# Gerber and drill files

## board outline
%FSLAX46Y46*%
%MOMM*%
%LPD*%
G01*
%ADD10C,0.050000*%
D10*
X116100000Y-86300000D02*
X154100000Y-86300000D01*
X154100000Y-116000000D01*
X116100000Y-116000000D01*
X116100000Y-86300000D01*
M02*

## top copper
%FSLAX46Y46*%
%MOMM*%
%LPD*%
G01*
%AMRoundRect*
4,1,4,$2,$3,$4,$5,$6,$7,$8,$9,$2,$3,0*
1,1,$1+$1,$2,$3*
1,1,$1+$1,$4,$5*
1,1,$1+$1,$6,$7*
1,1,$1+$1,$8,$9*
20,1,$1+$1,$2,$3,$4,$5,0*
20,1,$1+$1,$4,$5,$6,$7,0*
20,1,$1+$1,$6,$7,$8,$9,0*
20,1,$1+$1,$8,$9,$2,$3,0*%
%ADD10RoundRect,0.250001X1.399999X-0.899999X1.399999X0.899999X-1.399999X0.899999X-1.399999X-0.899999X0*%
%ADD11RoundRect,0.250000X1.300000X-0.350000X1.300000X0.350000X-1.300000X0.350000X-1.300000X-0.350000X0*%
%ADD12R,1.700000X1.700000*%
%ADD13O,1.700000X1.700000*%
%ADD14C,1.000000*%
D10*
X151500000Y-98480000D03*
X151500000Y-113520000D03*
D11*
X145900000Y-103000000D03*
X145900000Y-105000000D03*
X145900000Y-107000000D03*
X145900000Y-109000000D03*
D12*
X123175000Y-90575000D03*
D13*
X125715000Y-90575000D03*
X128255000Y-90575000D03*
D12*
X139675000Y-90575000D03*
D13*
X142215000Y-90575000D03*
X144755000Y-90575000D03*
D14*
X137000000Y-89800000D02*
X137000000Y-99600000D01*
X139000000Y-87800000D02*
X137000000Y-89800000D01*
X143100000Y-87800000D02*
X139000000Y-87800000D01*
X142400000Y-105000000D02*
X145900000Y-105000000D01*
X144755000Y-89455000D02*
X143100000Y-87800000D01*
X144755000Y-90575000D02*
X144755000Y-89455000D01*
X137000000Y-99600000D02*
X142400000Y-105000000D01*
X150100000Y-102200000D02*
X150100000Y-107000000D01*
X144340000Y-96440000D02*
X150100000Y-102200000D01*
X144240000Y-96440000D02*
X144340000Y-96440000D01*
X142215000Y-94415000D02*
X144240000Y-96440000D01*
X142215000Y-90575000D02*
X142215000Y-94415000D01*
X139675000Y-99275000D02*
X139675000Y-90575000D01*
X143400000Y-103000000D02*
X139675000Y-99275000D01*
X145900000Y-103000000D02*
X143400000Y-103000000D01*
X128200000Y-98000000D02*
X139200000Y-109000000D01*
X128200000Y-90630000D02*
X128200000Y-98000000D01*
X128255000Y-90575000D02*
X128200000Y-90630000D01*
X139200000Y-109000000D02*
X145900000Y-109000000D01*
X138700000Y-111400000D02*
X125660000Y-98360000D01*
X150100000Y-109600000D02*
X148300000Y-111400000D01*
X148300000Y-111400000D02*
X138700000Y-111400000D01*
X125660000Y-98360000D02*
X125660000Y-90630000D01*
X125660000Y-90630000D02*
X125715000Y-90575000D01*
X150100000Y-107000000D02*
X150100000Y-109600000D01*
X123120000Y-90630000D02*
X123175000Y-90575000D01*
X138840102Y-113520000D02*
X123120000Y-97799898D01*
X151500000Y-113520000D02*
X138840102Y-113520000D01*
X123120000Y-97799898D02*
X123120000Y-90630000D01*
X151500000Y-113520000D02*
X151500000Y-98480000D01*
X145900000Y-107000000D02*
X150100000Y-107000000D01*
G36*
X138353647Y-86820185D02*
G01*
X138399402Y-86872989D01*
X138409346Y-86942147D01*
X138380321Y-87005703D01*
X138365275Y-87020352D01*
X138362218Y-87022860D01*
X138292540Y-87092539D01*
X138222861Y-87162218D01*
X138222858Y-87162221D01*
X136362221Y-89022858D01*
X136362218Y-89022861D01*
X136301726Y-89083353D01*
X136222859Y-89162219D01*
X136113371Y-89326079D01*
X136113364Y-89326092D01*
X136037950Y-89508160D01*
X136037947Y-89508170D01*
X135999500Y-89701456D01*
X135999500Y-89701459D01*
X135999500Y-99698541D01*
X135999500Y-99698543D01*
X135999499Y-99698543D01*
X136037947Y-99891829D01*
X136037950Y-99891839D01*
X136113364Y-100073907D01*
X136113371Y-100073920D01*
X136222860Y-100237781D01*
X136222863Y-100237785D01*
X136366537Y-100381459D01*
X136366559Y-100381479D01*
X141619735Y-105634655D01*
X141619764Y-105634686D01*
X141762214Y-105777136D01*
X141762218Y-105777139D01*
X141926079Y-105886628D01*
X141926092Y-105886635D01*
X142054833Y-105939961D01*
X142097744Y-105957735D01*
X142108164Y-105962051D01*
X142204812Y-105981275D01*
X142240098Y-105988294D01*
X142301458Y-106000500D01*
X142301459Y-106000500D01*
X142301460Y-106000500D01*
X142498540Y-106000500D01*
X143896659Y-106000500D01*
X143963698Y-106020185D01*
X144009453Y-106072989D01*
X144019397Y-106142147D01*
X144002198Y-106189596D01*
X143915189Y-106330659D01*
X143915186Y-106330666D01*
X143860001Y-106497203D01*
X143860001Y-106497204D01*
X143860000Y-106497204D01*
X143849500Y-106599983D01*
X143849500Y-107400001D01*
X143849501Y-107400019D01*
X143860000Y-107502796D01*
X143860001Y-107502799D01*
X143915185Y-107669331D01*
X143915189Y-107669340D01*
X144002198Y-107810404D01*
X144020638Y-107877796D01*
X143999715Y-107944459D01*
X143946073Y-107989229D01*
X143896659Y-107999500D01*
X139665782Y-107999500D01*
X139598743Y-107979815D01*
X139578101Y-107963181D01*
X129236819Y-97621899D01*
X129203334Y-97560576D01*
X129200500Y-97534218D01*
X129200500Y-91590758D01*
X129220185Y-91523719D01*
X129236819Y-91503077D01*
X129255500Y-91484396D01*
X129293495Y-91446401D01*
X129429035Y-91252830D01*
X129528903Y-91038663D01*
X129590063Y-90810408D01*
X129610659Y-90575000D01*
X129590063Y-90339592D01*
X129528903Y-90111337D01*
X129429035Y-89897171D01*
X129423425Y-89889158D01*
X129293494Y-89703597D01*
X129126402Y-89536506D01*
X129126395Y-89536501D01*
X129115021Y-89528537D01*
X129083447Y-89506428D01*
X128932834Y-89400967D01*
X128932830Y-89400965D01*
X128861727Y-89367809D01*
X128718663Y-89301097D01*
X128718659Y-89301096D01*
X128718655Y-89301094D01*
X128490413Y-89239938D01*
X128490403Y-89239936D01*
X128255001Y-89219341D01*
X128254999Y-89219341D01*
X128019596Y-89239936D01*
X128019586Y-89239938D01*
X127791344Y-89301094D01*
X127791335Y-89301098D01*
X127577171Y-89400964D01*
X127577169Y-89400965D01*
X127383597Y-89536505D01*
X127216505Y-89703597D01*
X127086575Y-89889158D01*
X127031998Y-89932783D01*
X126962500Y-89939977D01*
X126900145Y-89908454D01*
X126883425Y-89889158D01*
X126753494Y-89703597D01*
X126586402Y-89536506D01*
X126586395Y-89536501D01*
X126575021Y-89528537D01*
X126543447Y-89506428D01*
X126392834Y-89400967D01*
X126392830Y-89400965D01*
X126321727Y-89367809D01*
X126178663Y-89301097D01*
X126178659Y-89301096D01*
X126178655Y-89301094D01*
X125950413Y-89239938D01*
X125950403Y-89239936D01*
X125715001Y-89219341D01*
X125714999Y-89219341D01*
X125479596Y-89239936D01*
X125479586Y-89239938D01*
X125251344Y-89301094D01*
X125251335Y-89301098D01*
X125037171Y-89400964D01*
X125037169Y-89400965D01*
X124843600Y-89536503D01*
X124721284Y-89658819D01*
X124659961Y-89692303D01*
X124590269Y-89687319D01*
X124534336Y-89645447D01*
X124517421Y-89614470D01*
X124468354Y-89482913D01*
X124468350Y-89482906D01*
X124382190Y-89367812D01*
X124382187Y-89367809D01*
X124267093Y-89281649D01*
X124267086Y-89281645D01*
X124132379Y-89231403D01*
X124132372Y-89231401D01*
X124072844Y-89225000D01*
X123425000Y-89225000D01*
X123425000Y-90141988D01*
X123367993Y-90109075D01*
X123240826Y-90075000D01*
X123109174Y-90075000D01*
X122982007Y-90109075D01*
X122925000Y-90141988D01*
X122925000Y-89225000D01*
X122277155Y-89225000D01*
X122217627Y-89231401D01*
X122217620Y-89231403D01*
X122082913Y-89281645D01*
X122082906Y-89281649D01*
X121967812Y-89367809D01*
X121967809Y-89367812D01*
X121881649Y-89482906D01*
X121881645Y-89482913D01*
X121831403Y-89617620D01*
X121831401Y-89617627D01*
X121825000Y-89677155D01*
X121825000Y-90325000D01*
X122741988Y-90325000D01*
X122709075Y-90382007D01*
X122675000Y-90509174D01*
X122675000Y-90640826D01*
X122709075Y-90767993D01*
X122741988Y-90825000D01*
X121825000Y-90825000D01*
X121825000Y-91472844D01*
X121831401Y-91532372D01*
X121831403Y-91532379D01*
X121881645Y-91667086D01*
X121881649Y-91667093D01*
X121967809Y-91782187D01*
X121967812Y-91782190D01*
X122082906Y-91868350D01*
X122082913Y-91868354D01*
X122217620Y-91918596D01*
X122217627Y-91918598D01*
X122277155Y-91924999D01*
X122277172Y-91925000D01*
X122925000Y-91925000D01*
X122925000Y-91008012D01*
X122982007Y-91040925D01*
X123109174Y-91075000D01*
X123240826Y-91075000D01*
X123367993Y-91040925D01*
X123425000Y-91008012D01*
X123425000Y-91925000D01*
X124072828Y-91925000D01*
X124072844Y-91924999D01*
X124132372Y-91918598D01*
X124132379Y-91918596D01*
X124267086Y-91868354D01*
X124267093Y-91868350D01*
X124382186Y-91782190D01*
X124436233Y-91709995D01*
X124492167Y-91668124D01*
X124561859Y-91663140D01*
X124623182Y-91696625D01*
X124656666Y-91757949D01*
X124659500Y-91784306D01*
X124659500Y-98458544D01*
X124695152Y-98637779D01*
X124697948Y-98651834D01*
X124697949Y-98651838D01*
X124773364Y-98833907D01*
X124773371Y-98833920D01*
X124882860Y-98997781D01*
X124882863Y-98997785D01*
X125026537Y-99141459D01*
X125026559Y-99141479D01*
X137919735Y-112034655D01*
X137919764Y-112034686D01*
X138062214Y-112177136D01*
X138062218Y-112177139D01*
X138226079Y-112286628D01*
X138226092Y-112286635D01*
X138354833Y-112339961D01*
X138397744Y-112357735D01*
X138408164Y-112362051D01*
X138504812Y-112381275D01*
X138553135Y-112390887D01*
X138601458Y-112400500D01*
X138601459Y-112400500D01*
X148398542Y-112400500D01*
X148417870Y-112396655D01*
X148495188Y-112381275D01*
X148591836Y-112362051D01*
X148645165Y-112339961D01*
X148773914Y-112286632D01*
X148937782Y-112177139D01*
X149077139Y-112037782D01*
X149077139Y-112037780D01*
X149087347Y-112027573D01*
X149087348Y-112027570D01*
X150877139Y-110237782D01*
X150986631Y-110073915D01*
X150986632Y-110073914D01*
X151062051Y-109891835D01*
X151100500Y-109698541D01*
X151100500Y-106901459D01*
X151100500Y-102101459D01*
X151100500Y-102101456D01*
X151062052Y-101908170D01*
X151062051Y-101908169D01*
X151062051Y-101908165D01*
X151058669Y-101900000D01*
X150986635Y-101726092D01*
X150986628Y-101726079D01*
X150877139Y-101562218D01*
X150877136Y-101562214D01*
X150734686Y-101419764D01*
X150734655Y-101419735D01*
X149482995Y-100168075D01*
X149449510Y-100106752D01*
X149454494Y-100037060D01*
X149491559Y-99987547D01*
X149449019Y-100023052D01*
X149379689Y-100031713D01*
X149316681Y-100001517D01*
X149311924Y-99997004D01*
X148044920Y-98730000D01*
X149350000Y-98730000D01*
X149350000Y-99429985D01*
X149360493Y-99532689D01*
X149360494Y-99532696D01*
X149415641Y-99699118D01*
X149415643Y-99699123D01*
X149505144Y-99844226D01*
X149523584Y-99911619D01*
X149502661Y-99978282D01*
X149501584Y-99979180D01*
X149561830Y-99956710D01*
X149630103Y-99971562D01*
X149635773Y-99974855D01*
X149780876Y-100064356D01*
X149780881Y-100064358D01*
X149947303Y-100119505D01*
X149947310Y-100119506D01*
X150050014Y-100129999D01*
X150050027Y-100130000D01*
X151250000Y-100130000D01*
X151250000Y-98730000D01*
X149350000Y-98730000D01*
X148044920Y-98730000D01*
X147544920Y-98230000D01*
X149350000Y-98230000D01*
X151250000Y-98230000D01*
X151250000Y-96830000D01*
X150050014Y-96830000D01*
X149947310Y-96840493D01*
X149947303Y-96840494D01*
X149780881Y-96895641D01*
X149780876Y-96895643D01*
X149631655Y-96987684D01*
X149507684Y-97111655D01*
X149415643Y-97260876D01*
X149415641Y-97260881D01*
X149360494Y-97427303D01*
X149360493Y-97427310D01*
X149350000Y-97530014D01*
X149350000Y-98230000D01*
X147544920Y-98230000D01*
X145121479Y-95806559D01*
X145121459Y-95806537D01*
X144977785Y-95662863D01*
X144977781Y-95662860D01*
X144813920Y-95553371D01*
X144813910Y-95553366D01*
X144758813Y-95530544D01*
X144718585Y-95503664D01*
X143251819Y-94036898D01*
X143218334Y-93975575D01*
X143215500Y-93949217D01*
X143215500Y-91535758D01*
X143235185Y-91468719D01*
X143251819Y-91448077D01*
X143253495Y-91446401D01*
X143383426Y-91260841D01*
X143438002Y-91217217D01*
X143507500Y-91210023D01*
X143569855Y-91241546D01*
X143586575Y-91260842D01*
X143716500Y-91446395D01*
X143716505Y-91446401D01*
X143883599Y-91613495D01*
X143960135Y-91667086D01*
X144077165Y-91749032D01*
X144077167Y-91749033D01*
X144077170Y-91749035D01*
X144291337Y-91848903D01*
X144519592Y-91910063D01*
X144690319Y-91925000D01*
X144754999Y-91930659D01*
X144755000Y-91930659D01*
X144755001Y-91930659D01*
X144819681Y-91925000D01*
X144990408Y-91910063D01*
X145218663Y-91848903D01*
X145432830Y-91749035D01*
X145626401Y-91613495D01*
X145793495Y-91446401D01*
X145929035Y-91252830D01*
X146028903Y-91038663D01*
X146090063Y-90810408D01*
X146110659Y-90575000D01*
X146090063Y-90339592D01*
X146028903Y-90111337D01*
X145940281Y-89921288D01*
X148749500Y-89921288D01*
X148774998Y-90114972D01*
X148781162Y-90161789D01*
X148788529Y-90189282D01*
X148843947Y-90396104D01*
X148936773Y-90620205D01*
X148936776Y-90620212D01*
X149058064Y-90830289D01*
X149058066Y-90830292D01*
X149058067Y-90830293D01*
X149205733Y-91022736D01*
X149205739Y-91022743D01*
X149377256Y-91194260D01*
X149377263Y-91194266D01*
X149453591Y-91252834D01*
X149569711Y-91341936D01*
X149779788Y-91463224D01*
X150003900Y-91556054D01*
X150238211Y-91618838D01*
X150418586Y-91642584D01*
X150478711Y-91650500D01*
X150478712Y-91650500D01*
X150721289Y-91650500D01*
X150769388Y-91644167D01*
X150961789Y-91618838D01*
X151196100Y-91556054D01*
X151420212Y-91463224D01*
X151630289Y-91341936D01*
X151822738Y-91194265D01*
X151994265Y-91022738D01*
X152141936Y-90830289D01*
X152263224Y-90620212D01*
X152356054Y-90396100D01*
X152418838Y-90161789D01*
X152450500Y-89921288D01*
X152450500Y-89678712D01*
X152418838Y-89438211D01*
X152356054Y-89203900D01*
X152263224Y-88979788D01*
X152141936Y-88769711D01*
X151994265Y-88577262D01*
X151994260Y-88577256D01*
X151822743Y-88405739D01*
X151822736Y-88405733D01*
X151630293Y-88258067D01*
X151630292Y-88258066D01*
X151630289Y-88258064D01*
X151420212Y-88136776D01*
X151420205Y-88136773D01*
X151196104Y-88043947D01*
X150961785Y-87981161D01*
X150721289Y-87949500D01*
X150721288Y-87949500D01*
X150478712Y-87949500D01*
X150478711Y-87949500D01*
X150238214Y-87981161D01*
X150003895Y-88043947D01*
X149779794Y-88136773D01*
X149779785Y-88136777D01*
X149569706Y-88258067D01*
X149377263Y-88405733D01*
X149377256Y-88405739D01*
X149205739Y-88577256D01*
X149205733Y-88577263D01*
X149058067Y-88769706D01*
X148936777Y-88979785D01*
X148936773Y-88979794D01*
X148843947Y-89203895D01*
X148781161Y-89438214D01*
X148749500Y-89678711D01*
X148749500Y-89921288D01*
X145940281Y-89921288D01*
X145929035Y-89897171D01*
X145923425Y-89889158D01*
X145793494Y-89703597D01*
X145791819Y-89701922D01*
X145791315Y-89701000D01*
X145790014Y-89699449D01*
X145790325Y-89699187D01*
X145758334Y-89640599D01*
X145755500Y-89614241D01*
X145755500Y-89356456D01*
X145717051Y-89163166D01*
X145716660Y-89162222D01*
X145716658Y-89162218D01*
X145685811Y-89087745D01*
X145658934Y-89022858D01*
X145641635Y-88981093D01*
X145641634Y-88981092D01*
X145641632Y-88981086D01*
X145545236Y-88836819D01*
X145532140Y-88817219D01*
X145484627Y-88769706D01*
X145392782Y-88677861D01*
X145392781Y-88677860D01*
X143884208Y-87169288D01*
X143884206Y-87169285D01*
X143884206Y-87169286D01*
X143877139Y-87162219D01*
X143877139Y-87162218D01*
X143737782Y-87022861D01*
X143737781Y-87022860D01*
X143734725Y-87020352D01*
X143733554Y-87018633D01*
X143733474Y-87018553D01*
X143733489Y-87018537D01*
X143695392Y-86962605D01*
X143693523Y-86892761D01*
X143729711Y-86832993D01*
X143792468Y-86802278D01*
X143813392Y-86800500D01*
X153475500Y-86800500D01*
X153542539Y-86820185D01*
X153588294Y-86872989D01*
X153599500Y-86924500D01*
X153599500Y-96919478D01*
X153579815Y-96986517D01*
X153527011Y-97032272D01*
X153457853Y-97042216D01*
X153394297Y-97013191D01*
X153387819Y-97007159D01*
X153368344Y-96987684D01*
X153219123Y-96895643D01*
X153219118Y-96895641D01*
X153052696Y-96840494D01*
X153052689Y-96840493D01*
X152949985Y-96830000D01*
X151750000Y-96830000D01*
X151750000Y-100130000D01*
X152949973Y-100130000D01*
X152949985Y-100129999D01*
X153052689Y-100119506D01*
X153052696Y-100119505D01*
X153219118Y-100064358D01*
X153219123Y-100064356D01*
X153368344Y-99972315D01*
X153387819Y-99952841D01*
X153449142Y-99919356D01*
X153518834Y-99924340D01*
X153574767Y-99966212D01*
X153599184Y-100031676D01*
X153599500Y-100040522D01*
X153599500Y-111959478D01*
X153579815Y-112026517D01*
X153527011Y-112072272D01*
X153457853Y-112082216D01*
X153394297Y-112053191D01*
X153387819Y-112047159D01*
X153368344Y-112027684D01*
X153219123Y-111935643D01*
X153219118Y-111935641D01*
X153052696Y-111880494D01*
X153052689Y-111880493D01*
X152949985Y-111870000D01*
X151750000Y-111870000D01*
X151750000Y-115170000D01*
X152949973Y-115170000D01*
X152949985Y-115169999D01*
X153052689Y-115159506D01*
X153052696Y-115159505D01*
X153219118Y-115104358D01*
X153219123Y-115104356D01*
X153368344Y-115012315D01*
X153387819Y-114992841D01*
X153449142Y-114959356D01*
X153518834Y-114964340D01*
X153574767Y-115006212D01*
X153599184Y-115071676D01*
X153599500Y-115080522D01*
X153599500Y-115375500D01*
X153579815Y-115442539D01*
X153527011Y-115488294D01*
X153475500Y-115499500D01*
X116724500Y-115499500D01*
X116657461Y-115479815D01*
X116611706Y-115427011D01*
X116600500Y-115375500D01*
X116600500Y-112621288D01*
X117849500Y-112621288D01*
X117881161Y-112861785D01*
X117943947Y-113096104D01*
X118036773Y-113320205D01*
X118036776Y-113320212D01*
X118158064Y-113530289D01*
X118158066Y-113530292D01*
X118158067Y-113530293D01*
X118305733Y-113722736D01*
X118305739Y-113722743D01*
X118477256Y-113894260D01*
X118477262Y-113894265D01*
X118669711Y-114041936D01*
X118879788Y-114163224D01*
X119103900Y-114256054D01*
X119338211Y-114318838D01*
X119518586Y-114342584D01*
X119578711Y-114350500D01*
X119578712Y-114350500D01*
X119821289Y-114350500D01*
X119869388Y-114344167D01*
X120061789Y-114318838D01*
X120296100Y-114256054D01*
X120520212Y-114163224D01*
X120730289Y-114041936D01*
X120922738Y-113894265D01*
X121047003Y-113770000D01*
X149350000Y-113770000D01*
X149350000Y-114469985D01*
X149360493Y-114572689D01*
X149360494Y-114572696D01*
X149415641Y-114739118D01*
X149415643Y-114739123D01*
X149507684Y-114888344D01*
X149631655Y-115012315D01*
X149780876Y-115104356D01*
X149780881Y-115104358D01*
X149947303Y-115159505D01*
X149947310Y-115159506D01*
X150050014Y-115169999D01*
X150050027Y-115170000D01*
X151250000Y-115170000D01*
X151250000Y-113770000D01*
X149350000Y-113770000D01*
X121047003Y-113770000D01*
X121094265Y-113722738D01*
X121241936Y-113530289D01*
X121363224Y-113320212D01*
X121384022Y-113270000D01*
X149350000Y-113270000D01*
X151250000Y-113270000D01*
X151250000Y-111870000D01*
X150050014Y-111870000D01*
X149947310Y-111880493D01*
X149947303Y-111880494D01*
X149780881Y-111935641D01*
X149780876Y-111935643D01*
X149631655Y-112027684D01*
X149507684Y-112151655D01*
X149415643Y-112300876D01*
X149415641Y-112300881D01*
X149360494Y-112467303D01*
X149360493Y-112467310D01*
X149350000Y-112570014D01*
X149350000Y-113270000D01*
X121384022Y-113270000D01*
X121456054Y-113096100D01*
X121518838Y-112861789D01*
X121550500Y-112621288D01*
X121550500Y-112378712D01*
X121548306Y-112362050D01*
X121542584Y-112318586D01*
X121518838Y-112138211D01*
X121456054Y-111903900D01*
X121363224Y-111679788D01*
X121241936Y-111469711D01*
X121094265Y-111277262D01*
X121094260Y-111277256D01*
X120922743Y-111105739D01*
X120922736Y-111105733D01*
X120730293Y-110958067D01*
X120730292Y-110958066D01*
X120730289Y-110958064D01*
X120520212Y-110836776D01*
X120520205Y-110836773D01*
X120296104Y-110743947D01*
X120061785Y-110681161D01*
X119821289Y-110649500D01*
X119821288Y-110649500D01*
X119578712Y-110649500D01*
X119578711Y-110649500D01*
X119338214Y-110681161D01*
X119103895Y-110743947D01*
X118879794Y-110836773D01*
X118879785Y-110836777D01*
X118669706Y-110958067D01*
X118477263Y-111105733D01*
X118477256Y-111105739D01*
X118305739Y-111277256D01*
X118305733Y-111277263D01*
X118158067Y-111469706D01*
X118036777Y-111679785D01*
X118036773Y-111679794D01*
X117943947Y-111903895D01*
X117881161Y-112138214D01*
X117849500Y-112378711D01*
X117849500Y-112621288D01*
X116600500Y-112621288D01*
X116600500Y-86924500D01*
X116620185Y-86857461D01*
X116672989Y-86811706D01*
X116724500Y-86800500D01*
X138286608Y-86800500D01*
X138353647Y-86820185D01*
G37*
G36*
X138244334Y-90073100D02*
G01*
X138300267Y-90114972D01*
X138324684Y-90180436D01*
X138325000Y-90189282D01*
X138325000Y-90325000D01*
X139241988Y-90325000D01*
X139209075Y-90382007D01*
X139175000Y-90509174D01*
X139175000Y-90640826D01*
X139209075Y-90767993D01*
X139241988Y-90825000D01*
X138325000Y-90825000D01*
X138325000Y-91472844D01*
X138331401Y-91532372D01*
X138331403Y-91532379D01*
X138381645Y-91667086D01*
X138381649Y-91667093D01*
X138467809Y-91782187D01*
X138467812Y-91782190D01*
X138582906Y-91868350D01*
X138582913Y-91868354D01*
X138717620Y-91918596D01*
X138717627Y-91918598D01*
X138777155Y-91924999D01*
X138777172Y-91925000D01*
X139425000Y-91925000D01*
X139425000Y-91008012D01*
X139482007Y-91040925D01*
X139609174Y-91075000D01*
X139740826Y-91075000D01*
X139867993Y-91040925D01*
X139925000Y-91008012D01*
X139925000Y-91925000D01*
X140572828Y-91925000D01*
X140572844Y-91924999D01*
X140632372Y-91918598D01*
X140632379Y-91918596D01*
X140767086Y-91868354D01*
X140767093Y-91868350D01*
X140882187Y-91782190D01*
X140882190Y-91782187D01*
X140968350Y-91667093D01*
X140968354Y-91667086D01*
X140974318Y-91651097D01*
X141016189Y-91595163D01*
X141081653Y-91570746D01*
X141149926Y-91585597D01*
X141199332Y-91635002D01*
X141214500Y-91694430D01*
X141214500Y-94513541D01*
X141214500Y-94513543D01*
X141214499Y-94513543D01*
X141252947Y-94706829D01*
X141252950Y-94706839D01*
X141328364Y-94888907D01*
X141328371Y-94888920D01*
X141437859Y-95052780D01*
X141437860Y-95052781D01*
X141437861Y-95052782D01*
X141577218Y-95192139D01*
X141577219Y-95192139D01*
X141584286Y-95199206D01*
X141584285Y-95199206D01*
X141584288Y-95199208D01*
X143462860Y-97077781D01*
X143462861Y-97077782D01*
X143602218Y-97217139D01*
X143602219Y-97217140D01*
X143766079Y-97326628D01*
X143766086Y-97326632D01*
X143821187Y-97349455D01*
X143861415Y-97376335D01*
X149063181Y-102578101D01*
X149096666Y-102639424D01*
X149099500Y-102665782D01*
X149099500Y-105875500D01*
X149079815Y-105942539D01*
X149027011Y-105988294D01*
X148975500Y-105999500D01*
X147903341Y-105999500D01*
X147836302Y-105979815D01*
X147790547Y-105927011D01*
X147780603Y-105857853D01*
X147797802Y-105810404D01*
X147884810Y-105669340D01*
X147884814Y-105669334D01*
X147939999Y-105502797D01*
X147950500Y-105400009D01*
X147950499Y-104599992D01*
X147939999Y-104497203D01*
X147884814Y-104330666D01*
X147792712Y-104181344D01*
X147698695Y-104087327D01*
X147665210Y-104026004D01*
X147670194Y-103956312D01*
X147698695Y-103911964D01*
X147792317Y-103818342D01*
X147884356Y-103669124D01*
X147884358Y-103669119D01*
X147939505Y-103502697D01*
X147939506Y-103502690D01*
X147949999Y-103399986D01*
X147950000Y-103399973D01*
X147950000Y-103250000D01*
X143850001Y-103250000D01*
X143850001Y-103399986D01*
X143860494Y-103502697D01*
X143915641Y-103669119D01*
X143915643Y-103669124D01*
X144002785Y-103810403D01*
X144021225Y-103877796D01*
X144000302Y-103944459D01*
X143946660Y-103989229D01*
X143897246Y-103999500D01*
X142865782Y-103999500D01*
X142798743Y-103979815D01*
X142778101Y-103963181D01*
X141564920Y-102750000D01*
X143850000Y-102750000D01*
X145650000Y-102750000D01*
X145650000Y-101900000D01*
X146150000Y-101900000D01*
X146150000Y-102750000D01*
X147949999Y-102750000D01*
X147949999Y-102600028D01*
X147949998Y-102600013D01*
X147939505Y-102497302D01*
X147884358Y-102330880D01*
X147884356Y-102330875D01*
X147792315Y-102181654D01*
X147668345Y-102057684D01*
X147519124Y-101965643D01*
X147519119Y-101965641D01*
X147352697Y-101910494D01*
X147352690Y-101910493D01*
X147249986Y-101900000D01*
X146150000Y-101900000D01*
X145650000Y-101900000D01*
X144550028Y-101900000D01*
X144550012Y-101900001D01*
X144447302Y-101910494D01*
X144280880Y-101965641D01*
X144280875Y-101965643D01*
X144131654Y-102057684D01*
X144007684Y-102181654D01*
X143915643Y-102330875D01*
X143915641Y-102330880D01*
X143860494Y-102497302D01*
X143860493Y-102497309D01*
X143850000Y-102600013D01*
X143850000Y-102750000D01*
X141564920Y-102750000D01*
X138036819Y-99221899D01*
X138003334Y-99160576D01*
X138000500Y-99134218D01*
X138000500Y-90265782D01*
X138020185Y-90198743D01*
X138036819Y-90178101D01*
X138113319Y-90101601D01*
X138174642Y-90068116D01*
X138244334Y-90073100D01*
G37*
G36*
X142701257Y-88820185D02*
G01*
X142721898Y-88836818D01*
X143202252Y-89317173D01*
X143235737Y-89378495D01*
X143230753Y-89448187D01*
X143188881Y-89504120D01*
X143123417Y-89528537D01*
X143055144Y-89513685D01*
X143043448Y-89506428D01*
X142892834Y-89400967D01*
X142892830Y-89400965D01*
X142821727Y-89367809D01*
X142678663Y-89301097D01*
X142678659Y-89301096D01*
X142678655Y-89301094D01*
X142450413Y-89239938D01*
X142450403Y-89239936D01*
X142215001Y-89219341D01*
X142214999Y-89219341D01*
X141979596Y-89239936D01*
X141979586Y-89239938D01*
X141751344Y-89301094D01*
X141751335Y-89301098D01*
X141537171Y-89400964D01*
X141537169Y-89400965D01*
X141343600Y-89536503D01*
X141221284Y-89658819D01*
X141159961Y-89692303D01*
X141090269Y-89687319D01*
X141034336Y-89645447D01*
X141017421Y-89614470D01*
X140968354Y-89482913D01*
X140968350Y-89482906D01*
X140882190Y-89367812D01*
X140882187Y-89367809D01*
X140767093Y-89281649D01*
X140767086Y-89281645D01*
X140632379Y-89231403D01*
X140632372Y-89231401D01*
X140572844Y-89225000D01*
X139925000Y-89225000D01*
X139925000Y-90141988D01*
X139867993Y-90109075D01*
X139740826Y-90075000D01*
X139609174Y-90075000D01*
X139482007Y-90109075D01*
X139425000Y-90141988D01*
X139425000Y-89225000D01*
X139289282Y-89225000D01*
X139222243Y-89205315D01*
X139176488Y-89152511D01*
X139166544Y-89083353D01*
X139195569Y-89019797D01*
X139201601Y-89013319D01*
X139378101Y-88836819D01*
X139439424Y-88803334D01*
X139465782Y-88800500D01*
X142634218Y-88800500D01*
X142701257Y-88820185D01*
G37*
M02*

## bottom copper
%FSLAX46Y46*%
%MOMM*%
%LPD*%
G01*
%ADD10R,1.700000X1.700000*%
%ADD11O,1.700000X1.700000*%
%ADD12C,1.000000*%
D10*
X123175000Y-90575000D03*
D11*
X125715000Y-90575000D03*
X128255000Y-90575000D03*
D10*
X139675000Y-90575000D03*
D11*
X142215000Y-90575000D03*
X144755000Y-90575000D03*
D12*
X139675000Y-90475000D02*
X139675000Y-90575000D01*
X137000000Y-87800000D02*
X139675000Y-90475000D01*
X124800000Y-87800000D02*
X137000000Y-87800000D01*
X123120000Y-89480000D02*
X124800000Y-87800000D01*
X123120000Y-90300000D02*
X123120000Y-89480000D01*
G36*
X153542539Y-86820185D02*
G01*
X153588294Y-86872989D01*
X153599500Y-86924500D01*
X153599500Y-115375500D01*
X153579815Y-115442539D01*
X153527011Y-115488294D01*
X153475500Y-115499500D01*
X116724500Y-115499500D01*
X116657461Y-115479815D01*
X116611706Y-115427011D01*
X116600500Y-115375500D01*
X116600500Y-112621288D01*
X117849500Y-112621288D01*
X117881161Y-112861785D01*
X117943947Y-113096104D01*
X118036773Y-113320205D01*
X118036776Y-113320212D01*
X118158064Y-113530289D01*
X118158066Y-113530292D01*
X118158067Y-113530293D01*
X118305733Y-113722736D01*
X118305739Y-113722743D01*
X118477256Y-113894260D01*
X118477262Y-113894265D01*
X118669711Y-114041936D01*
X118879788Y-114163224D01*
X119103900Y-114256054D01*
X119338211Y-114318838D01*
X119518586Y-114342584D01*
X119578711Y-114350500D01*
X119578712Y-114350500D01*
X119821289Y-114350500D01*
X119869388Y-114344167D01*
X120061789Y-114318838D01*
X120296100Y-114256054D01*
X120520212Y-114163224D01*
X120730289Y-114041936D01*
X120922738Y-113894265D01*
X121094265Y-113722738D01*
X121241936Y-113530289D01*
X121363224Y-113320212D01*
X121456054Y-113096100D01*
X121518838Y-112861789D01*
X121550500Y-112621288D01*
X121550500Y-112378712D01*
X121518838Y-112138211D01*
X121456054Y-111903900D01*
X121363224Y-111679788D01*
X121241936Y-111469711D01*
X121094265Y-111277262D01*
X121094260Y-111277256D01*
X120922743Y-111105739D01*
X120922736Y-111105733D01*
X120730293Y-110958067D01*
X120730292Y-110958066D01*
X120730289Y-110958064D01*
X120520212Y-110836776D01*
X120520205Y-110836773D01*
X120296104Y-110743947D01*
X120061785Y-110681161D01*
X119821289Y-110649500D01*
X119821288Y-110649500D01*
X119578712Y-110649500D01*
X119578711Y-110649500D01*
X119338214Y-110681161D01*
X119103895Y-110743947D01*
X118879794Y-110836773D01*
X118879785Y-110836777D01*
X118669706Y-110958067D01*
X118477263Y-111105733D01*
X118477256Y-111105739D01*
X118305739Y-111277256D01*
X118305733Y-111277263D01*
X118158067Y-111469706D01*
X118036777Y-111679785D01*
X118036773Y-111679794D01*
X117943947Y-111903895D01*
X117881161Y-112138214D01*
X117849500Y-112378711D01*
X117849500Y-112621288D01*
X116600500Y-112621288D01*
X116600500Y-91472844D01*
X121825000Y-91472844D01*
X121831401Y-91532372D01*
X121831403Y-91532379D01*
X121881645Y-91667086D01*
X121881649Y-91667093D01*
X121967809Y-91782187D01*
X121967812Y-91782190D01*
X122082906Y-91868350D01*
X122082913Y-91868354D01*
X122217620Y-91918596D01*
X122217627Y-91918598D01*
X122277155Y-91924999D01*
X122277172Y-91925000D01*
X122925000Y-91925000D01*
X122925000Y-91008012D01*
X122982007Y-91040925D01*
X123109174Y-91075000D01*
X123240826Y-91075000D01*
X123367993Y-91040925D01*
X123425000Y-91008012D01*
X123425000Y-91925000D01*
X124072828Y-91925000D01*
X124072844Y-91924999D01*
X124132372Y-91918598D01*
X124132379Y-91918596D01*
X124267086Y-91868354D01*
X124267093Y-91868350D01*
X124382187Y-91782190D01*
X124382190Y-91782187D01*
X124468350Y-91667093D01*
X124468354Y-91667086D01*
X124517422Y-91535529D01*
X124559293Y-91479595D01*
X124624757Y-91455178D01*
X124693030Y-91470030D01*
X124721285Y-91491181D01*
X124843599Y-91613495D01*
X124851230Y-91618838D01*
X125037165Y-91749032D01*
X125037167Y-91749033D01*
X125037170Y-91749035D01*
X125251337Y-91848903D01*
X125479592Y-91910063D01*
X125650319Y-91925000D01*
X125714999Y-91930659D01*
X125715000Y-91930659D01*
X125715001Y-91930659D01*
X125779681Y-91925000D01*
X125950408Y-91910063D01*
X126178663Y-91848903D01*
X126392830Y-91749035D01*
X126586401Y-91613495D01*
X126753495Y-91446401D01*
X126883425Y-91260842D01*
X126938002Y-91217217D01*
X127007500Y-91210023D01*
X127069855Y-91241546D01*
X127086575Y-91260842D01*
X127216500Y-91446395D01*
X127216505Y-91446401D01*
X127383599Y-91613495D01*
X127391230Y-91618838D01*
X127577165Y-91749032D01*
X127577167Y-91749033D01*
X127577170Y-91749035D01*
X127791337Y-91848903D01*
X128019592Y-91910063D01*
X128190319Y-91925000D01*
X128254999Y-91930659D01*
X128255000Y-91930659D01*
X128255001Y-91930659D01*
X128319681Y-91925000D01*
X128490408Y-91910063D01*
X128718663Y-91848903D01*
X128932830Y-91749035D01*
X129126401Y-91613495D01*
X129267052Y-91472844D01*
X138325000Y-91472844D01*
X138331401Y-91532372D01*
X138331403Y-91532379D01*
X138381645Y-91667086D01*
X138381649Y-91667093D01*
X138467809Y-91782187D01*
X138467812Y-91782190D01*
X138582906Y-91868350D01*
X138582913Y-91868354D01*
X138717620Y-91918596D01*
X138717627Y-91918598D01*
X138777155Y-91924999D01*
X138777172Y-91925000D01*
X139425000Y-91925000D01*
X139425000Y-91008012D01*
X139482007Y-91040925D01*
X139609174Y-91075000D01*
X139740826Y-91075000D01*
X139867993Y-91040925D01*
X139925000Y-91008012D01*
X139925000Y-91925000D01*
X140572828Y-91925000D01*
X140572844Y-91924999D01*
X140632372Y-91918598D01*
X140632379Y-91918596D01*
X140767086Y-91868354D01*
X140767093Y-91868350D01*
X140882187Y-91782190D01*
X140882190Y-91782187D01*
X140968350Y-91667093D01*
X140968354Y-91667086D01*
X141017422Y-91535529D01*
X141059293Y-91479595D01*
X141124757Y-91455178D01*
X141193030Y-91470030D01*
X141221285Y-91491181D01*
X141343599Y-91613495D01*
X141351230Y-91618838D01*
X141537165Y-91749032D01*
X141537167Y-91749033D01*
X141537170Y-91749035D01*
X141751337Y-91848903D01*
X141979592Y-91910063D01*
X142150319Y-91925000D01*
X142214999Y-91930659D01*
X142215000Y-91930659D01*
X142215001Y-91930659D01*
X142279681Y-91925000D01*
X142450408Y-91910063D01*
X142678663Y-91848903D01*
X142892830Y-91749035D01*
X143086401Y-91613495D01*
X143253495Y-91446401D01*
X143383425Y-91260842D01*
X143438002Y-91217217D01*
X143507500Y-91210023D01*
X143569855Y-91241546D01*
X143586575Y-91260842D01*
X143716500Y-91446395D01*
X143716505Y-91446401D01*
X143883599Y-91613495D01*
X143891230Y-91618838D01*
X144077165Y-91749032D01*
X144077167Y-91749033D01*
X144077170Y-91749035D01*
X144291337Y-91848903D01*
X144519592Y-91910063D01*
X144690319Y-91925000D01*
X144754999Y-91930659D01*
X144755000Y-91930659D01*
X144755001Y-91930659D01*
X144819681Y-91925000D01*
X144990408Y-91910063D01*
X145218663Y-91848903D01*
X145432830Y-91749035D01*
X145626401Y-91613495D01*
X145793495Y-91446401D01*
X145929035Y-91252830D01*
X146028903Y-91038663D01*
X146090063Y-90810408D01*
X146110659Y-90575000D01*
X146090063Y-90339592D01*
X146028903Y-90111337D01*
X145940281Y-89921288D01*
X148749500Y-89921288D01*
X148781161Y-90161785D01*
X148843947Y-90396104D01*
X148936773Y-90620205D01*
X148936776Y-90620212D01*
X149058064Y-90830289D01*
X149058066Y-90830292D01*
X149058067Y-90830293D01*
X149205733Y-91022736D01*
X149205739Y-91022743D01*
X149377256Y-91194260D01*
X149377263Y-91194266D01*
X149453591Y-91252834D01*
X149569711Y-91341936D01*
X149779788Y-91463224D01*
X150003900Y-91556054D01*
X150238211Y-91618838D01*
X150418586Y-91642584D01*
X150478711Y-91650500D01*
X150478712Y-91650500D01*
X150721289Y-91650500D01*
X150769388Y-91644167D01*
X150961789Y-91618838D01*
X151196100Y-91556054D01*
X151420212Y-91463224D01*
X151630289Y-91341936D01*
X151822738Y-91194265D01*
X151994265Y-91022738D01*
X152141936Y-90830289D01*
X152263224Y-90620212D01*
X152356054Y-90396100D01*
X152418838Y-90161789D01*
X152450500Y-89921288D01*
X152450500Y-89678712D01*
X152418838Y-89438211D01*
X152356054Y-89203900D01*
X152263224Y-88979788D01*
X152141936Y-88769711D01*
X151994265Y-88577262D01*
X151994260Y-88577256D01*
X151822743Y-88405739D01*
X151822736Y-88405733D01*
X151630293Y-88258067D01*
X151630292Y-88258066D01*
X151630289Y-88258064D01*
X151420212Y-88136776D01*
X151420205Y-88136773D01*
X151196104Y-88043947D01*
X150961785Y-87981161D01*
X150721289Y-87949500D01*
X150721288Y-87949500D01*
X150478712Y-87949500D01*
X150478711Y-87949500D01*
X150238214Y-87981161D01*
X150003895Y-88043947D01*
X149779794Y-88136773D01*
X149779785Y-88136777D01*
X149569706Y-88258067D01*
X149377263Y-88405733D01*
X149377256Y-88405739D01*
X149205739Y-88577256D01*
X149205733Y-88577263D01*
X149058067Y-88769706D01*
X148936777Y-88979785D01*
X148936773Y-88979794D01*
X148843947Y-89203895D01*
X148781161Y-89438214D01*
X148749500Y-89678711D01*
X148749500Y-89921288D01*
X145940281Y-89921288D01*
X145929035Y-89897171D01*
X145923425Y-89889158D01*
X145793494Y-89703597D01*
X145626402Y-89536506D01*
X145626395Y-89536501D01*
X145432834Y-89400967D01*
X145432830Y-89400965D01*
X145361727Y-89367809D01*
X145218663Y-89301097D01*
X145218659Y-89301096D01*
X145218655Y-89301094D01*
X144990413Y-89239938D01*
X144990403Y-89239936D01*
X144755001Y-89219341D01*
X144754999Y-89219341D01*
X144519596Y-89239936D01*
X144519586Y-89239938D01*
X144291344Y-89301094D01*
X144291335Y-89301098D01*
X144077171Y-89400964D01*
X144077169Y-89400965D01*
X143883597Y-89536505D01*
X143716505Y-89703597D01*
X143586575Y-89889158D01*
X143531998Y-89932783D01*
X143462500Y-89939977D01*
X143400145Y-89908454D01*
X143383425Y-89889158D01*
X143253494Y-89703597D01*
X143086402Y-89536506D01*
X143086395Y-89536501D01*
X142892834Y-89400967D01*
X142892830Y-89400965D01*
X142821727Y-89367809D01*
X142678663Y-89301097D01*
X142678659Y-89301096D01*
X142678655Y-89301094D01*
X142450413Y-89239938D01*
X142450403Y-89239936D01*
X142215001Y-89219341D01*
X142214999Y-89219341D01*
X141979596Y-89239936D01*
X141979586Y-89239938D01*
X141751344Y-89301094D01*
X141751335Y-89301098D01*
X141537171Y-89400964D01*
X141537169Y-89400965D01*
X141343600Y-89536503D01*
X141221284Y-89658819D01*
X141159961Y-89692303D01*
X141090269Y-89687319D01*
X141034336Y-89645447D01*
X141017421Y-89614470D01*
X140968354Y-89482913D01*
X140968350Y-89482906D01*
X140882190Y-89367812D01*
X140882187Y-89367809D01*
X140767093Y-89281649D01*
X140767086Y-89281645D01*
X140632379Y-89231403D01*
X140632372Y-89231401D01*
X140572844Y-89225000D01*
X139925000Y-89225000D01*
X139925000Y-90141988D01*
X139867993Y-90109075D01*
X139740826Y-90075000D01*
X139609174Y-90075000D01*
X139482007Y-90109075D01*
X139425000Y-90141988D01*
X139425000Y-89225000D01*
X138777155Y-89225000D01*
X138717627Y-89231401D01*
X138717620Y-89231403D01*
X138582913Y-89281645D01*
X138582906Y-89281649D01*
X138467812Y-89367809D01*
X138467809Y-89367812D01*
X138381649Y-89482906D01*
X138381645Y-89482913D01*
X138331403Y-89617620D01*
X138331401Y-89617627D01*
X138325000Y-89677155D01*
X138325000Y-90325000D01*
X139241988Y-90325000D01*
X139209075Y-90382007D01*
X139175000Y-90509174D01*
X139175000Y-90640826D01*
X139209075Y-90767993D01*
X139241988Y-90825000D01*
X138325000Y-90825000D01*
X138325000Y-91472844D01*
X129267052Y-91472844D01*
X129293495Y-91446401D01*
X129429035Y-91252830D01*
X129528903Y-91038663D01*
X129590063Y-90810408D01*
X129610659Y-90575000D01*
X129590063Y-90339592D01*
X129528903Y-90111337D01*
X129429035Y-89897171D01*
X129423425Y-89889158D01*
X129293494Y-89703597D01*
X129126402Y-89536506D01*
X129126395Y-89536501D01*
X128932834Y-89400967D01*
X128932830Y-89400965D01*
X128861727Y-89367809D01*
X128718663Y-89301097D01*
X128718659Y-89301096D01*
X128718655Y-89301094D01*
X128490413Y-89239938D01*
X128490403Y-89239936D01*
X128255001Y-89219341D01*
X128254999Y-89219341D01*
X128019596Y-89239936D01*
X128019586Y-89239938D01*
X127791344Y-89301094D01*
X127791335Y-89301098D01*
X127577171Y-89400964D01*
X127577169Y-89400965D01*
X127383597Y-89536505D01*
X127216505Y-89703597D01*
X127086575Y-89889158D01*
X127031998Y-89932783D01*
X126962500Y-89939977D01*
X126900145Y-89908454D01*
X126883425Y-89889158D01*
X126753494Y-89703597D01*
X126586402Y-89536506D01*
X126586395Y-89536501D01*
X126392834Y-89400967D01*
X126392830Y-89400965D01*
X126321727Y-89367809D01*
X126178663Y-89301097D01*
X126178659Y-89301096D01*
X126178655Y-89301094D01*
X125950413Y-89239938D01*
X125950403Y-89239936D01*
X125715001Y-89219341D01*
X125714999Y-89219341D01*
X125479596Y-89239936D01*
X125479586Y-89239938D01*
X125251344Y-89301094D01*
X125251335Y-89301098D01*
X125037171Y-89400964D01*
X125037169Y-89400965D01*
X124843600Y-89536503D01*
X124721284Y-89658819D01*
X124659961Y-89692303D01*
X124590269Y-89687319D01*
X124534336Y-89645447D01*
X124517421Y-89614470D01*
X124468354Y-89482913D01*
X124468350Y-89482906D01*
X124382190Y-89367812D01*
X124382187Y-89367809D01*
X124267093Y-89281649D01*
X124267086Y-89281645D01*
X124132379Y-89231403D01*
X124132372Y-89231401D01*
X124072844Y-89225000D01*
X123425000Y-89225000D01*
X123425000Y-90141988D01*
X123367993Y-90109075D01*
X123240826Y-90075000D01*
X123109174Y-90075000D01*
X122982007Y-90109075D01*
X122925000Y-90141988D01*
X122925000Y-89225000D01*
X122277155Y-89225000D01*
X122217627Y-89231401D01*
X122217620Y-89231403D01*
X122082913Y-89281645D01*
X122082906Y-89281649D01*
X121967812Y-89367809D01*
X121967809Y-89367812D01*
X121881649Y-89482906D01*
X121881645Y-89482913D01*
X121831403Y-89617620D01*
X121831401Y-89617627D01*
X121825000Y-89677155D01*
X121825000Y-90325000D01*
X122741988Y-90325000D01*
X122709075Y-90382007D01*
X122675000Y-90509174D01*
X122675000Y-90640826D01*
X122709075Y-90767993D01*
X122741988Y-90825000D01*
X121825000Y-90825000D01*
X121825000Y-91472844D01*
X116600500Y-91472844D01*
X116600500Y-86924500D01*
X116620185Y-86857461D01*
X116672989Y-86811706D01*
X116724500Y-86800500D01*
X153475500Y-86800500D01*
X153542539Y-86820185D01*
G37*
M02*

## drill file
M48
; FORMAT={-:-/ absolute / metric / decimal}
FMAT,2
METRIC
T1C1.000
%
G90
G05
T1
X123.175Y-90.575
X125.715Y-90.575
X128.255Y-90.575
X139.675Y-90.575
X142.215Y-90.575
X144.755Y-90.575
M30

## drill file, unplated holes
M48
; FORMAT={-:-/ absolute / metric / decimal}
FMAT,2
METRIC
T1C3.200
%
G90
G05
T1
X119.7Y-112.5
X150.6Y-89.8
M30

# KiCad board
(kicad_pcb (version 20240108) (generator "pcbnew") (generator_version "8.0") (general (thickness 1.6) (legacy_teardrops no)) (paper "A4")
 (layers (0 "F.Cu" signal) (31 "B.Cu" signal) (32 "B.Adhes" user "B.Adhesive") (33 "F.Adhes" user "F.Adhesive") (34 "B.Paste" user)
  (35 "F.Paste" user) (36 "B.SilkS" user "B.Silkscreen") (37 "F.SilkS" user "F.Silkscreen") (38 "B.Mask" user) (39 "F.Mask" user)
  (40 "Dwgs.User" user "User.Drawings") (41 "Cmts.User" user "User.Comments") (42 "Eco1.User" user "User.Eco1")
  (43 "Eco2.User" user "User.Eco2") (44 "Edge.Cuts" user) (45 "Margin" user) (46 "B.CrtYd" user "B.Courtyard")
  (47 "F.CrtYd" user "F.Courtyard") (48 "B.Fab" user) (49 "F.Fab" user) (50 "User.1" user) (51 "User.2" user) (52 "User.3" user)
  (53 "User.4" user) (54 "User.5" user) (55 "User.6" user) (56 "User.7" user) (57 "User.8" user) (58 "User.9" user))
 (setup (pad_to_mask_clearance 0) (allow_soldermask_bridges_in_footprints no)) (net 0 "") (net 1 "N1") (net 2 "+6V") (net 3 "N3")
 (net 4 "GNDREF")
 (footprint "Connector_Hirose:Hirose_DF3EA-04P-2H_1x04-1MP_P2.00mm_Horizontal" (layer "F.Cu") (at 148.75 106 90)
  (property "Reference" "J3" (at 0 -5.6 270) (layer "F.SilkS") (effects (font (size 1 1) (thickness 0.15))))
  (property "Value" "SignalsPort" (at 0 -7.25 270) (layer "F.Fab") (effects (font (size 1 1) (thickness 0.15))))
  (pad "1" smd roundrect (at -3 -2.85 90) (size 1.2 3.1) (layers "F.Cu" "F.Paste" "F.Mask") (roundrect_rratio 0.208333) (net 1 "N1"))
  (pad "2" smd roundrect (at -1 -2.85 90) (size 1.2 3.1) (layers "F.Cu" "F.Paste" "F.Mask") (roundrect_rratio 0.208333) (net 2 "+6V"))
  (pad "3" smd roundrect (at 1 -2.85 90) (size 1.2 3.1) (layers "F.Cu" "F.Paste" "F.Mask") (roundrect_rratio 0.208333) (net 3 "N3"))
  (pad "4" smd roundrect (at 3 -2.85 90) (size 1.2 3.1) (layers "F.Cu" "F.Paste" "F.Mask") (roundrect_rratio 0.208333) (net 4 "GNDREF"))
  (pad "MP" smd roundrect (at -7.52 2.75 90) (size 2.3 3.3) (layers "F.Cu" "F.Paste" "F.Mask") (roundrect_rratio 0.108696) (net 4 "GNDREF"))
  (pad "MP" smd roundrect (at 7.52 2.75 90) (size 2.3 3.3) (layers "F.Cu" "F.Paste" "F.Mask") (roundrect_rratio 0.108696) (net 4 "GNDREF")))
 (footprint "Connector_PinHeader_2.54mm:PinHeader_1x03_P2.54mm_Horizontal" (layer "F.Cu") (at 123.175 90.575 90)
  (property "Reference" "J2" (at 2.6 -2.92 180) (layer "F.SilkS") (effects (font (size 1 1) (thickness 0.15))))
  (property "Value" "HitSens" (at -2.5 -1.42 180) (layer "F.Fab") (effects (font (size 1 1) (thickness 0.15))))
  (pad "1" thru_hole rect (at 0 0 90) (size 1.7 1.7) (drill 1) (layers "*.Cu" "*.Mask") (remove_unused_layers no) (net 4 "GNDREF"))
  (pad "2" thru_hole oval (at 0 2.54 90) (size 1.7 1.7) (drill 1) (layers "*.Cu" "*.Mask") (remove_unused_layers no) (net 2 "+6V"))
  (pad "3" thru_hole oval (at 0 5.08 90) (size 1.7 1.7) (drill 1) (layers "*.Cu" "*.Mask") (remove_unused_layers no) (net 1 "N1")))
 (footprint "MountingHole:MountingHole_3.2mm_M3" (layer "F.Cu") (at 150.6 89.8)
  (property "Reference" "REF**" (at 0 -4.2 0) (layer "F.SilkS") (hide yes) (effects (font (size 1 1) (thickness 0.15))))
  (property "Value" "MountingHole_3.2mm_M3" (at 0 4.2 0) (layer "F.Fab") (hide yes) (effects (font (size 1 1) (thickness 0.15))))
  (pad "" np_thru_hole circle (at 0 0) (size 3.2 3.2) (drill 3.2) (layers "F&B.Cu" "*.Mask")))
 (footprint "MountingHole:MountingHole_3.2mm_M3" (layer "F.Cu") (at 119.7 112.5)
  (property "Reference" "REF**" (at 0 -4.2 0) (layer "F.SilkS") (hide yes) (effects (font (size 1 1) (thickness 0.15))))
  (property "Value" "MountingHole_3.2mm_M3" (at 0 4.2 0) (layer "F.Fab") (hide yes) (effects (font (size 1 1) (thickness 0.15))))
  (pad "" np_thru_hole circle (at 0 0) (size 3.2 3.2) (drill 3.2) (layers "*.Cu" "*.Mask")))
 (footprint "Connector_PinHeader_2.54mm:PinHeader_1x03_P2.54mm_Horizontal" (layer "F.Cu") (at 139.675 90.575 90)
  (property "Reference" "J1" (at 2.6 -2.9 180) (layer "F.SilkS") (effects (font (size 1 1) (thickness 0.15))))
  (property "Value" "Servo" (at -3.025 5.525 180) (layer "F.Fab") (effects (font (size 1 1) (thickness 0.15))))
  (pad "1" thru_hole rect (at 0 0 90) (size 1.7 1.7) (drill 1) (layers "*.Cu" "*.Mask") (remove_unused_layers no) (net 4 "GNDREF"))
  (pad "2" thru_hole oval (at 0 2.54 90) (size 1.7 1.7) (drill 1) (layers "*.Cu" "*.Mask") (remove_unused_layers no) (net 2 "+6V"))
  (pad "3" thru_hole oval (at 0 5.08 90) (size 1.7 1.7) (drill 1) (layers "*.Cu" "*.Mask") (remove_unused_layers no) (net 3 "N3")))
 (gr_rect (start 116.1 86.3) (end 154.1 116) (stroke (width 0.05) (type default)) (fill none) (layer "Edge.Cuts"))
 (segment (start 144.34 96.44) (end 150.1 102.2) (width 1) (layer "F.Cu") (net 2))
 (segment (start 138.7 111.4) (end 125.66 98.36) (width 1) (layer "F.Cu") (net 2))
 (segment (start 142.215 94.415) (end 144.24 96.44) (width 1) (layer "F.Cu") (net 2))
 (segment (start 125.66 90.63) (end 125.715 90.575) (width 1) (layer "F.Cu") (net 2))
 (segment (start 150.1 109.6) (end 148.3 111.4) (width 1) (layer "F.Cu") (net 2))
 (segment (start 145.9 107) (end 150.1 107) (width 1) (layer "F.Cu") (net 2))
 (segment (start 150.1 107) (end 150.1 109.6) (width 1) (layer "F.Cu") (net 2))
 (segment (start 125.66 98.36) (end 125.66 90.63) (width 1) (layer "F.Cu") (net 2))
 (segment (start 142.215 90.575) (end 142.215 94.415) (width 1) (layer "F.Cu") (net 2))
 (segment (start 148.3 111.4) (end 138.7 111.4) (width 1) (layer "F.Cu") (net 2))
 (segment (start 144.24 96.44) (end 144.34 96.44) (width 1) (layer "F.Cu") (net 2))
 (segment (start 150.1 102.2) (end 150.1 107) (width 1) (layer "F.Cu") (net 2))
 (segment (start 139.675 99.275) (end 139.675 90.575) (width 1) (layer "F.Cu") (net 4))
 (segment (start 151.5 113.52) (end 138.840102 113.52) (width 1) (layer "F.Cu") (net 4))
 (segment (start 138.840102 113.52) (end 123.12 97.799898) (width 1) (layer "F.Cu") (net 4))
 (segment (start 123.12 97.799898) (end 123.12 90.63) (width 1) (layer "F.Cu") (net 4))
 (segment (start 123.12 90.63) (end 123.175 90.575) (width 1) (layer "F.Cu") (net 4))
 (segment (start 151.5 113.52) (end 151.5 98.48) (width 1) (layer "F.Cu") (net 4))
 (segment (start 143.4 103) (end 139.675 99.275) (width 1) (layer "F.Cu") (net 4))
 (segment (start 145.9 103) (end 143.4 103) (width 1) (layer "F.Cu") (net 4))
 (segment (start 123.12 90.3) (end 123.12 89.48) (width 1) (layer "B.Cu") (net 4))
 (segment (start 123.12 89.48) (end 124.8 87.8) (width 1) (layer "B.Cu") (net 4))
 (segment (start 139.675 90.475) (end 139.675 90.575) (width 1) (layer "B.Cu") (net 4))
 (segment (start 124.8 87.8) (end 137 87.8) (width 1) (layer "B.Cu") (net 4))
 (segment (start 137 87.8) (end 139.675 90.475) (width 1) (layer "B.Cu") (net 4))
 (segment (start 137 99.6) (end 142.4 105) (width 1) (layer "F.Cu") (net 3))
 (segment (start 144.755 89.455) (end 143.1 87.8) (width 1) (layer "F.Cu") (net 3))
 (segment (start 143.1 87.8) (end 139 87.8) (width 1) (layer "F.Cu") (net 3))
 (segment (start 139 87.8) (end 137 89.8) (width 1) (layer "F.Cu") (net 3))
 (segment (start 144.755 90.575) (end 144.755 89.455) (width 1) (layer "F.Cu") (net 3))
 (segment (start 142.4 105) (end 145.9 105) (width 1) (layer "F.Cu") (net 3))
 (segment (start 137 89.8) (end 137 99.6) (width 1) (layer "F.Cu") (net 3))
 (segment (start 128.255 90.575) (end 128.2 90.63) (width 1) (layer "F.Cu") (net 1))
 (segment (start 128.2 98) (end 139.2 109) (width 1) (layer "F.Cu") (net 1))
 (segment (start 128.2 90.63) (end 128.2 98) (width 1) (layer "F.Cu") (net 1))
 (segment (start 139.2 109) (end 145.9 109) (width 1) (layer "F.Cu") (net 1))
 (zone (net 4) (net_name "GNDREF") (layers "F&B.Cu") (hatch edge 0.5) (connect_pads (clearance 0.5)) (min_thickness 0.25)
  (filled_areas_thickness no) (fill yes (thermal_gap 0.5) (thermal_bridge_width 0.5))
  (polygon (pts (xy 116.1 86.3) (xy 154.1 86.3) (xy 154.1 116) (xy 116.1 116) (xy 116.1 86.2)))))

